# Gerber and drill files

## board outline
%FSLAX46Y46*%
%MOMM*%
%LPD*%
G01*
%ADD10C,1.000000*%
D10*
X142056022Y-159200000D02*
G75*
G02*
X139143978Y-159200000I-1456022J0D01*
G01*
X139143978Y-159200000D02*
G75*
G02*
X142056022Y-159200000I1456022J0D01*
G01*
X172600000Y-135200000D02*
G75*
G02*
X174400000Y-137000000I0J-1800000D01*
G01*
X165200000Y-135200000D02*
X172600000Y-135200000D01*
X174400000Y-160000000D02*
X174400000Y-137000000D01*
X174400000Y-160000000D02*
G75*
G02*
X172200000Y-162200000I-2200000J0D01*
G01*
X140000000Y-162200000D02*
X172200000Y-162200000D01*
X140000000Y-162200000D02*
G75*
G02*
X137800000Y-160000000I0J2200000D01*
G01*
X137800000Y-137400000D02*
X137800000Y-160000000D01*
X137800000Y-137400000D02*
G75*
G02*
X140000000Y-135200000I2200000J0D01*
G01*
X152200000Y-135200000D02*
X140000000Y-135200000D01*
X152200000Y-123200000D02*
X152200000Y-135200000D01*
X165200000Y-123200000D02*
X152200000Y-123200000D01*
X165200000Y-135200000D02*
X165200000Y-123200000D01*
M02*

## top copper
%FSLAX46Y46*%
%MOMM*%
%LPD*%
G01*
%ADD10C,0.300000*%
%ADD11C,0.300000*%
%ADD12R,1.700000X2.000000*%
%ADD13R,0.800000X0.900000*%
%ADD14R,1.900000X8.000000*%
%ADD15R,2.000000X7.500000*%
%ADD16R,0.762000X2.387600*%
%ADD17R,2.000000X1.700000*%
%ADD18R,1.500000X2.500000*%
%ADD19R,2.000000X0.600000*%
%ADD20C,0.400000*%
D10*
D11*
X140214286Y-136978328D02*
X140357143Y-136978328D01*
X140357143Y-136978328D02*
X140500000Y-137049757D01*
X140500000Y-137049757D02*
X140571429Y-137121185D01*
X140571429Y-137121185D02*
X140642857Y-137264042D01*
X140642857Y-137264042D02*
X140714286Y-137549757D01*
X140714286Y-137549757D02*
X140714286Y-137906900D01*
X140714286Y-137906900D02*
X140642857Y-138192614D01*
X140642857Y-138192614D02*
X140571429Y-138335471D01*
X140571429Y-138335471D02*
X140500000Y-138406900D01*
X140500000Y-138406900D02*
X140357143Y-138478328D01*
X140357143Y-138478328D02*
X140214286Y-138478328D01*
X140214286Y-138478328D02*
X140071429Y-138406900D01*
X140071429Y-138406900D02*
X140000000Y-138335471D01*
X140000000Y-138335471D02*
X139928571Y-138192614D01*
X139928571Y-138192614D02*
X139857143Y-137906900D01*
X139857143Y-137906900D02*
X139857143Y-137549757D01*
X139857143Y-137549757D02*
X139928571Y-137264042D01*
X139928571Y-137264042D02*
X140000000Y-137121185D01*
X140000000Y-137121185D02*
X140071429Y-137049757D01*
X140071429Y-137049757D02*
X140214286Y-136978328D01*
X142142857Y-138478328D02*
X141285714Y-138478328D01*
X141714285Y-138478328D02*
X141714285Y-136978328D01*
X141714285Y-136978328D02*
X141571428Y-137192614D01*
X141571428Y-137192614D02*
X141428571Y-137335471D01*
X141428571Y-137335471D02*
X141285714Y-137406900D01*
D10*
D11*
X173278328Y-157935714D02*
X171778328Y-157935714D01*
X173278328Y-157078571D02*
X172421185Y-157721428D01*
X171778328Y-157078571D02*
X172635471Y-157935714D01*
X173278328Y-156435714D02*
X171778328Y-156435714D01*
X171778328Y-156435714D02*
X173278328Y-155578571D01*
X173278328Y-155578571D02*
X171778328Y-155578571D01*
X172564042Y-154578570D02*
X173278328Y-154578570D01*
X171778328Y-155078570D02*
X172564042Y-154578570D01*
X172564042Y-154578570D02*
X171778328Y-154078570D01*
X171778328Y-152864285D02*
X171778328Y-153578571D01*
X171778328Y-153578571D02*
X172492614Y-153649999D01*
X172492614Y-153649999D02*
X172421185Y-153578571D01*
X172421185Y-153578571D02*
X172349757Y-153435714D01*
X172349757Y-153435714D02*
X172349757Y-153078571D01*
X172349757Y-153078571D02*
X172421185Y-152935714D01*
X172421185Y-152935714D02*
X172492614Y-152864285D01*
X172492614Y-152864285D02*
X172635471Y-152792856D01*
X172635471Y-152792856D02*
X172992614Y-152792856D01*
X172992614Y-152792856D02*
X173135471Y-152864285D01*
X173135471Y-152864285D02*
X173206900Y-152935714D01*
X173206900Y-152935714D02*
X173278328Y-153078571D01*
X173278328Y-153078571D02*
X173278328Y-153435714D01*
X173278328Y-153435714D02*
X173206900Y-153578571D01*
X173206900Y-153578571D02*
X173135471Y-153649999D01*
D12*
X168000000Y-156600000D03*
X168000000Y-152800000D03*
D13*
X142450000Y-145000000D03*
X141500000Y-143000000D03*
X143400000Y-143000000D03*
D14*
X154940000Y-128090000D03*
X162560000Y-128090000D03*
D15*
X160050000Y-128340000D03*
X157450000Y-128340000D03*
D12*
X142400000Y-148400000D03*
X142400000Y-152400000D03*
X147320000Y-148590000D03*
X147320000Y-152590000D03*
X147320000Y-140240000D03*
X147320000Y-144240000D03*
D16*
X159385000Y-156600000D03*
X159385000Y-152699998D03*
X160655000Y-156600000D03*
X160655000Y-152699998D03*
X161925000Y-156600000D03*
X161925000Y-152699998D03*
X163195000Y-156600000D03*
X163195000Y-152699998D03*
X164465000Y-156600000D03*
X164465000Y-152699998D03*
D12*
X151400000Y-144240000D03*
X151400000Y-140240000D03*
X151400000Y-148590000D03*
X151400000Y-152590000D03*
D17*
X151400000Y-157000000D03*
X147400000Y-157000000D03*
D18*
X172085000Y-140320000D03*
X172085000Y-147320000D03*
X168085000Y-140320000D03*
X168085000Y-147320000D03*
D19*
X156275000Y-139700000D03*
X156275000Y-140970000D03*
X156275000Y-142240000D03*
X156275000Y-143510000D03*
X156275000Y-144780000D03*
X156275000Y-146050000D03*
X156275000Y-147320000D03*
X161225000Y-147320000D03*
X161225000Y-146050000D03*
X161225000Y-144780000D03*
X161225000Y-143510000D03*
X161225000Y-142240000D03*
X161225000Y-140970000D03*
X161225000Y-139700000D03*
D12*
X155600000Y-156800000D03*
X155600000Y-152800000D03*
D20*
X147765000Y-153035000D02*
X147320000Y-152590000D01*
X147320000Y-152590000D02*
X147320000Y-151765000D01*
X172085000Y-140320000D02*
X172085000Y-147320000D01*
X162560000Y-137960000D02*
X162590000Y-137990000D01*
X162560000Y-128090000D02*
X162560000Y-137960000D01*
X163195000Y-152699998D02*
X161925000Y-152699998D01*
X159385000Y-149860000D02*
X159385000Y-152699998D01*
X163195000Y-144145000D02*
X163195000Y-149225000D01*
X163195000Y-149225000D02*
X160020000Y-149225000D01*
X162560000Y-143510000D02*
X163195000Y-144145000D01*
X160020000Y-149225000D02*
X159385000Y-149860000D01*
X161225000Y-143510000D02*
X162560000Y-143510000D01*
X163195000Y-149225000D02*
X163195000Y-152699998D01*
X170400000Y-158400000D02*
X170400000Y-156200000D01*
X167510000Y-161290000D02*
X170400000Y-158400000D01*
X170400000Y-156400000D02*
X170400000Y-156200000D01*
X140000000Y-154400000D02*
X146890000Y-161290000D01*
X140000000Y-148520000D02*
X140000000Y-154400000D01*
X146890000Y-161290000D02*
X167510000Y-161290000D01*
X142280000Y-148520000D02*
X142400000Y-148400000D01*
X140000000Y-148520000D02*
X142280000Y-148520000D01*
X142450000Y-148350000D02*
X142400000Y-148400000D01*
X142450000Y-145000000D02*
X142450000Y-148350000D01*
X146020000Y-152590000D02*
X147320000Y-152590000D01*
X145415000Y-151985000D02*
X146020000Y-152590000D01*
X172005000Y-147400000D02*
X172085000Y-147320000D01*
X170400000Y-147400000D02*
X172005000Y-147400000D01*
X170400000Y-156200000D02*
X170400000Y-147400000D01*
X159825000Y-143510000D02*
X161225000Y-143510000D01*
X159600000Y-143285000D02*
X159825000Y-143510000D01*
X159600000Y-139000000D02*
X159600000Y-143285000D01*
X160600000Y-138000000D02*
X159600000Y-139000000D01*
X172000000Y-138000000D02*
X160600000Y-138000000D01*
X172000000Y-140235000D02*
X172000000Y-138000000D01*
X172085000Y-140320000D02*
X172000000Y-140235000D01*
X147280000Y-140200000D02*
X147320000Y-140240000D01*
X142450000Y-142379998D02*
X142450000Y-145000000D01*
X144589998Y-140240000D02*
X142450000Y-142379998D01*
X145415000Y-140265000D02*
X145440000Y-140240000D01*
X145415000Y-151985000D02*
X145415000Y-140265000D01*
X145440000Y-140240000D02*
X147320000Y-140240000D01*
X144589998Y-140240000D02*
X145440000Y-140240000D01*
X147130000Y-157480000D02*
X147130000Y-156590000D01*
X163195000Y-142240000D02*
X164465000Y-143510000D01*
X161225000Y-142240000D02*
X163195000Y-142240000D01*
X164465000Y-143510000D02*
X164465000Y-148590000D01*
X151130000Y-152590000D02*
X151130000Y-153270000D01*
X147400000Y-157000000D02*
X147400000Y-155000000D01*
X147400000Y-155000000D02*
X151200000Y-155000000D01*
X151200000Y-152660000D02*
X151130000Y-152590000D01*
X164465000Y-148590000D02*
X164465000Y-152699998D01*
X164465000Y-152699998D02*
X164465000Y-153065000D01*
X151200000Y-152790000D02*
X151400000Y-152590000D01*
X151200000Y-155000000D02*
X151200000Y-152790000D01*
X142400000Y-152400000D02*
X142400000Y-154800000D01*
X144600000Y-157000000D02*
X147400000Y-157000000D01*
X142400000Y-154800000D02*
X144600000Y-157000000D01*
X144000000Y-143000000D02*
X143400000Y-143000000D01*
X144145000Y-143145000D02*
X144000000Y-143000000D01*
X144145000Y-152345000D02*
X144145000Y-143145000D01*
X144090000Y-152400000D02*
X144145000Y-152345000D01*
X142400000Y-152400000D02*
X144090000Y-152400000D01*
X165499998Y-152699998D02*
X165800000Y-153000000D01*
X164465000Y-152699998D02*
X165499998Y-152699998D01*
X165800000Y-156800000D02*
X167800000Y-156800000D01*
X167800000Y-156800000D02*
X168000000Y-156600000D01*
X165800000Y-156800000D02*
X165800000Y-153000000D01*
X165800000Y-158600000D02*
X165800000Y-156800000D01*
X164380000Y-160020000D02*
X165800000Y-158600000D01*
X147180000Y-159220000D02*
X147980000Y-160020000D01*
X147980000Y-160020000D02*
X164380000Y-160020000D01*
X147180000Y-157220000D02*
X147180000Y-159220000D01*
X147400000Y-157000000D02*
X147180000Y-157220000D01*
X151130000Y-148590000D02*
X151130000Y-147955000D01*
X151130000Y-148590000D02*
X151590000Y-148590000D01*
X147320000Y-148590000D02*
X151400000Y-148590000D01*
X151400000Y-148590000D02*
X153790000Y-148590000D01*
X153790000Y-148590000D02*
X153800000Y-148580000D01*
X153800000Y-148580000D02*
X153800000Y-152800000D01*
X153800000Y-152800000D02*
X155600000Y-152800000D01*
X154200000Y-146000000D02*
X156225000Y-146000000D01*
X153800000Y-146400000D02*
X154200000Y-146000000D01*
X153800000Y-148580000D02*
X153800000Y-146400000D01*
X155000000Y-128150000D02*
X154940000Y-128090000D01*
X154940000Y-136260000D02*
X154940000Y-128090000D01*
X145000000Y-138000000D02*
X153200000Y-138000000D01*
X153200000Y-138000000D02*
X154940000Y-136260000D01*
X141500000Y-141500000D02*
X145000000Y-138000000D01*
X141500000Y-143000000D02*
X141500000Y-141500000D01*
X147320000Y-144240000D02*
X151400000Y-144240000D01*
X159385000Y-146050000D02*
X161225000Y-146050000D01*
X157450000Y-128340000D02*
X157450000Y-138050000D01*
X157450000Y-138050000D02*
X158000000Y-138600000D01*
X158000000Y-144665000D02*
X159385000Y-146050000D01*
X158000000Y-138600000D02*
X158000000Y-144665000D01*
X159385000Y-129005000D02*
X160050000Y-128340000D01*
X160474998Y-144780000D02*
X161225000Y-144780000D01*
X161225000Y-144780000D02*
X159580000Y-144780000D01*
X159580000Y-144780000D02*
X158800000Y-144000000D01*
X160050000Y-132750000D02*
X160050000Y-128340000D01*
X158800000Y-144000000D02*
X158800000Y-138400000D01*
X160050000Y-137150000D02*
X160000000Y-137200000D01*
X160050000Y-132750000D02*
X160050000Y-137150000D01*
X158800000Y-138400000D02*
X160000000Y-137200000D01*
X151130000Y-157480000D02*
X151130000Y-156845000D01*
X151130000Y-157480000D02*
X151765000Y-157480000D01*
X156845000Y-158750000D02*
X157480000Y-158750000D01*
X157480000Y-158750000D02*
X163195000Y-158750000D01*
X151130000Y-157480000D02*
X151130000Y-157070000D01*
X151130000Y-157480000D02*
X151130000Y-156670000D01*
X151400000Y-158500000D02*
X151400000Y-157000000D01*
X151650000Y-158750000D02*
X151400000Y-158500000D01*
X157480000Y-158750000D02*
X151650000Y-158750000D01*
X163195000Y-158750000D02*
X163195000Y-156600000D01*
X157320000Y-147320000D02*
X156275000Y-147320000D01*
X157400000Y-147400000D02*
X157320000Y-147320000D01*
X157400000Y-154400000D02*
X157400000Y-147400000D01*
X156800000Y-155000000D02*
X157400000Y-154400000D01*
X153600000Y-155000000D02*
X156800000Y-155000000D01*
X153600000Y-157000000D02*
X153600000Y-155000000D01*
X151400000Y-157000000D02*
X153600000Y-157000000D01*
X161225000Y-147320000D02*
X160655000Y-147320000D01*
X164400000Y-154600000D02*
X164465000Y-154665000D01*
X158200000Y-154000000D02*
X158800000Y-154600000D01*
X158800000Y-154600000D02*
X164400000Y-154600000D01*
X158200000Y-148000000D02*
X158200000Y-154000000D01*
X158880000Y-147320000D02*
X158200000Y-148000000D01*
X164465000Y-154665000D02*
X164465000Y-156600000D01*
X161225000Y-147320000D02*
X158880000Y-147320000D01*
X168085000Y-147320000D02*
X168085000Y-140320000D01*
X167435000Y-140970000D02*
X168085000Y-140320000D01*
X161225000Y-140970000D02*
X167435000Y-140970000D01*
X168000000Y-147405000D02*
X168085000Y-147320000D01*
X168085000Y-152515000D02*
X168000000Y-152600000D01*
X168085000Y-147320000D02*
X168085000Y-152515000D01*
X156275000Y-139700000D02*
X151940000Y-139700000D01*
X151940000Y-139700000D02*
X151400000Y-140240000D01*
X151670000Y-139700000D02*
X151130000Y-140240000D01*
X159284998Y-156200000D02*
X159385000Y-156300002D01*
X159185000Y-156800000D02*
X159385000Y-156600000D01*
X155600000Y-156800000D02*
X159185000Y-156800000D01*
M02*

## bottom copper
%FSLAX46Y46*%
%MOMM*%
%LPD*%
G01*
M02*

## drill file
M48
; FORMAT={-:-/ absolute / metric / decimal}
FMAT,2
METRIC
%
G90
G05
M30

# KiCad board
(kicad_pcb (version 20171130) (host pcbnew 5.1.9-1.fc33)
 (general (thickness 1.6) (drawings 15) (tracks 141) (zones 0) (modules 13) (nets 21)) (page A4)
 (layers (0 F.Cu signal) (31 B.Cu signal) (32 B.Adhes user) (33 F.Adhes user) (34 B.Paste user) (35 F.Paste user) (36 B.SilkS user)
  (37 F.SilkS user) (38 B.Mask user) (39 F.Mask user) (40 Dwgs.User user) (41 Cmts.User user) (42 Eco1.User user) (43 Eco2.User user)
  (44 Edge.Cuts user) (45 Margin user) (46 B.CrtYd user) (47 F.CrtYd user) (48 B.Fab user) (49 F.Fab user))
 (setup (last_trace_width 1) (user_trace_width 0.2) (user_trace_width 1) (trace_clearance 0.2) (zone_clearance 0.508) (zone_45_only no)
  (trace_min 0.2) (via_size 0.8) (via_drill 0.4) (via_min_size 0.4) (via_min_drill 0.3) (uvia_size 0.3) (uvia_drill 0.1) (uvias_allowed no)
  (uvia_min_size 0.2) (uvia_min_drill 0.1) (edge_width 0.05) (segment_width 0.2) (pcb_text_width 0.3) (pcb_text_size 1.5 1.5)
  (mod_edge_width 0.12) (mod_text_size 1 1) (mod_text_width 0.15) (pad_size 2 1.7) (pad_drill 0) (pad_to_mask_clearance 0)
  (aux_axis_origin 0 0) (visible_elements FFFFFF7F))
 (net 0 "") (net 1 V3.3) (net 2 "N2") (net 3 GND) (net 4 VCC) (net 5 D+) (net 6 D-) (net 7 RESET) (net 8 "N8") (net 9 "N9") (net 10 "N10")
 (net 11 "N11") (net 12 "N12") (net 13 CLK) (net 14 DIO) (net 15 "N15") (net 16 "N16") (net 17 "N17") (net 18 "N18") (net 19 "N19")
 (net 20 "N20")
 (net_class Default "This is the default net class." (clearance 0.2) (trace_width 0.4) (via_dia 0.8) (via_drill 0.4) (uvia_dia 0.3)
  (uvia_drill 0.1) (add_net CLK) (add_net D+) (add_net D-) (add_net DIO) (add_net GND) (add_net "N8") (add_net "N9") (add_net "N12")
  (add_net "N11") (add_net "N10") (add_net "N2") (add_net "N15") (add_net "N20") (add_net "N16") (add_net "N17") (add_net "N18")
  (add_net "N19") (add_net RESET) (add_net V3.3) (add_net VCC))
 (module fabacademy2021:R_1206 (layer F.Cu) (at 168 154.6 90)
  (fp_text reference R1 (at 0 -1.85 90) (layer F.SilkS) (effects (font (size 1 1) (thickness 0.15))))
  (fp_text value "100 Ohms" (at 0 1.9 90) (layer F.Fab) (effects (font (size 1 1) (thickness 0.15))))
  (pad 1 smd rect (at -2 0 90) (size 2 1.7) (layers F.Cu F.Paste F.Mask) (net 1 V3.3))
  (pad 2 smd rect (at 1.8 0 90) (size 2 1.7) (layers F.Cu F.Paste F.Mask) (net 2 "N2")))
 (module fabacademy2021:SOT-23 (layer F.Cu) (at 142.45 144 270)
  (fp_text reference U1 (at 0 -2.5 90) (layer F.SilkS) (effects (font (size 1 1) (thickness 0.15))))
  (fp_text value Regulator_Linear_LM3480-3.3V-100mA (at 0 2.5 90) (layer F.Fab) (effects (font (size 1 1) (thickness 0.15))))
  (pad 3 smd rect (at 1 0 270) (size 0.9 0.8) (layers F.Cu F.Paste F.Mask) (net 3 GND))
  (pad 2 smd rect (at -1 0.95 270) (size 0.9 0.8) (layers F.Cu F.Paste F.Mask) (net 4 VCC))
  (pad 1 smd rect (at -1 -0.95 270) (size 0.9 0.8) (layers F.Cu F.Paste F.Mask) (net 1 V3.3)))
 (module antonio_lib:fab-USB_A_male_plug (layer F.Cu) (at 158.75 123.19 180)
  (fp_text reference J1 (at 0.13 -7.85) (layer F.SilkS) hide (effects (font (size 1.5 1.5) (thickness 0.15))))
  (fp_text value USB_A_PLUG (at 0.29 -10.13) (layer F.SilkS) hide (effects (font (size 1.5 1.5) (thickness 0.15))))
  (pad 1 connect rect (at 3.81 -4.9 180) (size 1.9 8) (layers F.Cu F.Mask) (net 4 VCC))
  (pad 4 connect rect (at -3.81 -4.9 180) (size 1.9 8) (layers F.Cu F.Mask) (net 3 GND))
  (pad 3 connect rect (at -1.3 -5.15 180) (size 2 7.5) (layers F.Cu F.Mask) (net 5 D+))
  (pad 2 connect rect (at 1.3 -5.15 180) (size 2 7.5) (layers F.Cu F.Mask) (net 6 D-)))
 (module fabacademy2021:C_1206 (layer F.Cu) (at 142.4 150.4 90)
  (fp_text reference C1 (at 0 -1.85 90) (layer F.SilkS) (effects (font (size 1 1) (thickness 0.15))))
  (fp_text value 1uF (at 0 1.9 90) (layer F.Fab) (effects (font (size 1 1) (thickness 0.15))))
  (pad 2 smd rect (at 2 0 90) (size 2 1.7) (layers F.Cu F.Paste F.Mask) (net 3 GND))
  (pad 1 smd rect (at -2 0 90) (size 2 1.7) (layers F.Cu F.Paste F.Mask) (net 1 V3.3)))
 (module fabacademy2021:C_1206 (layer F.Cu) (at 147.32 150.59 270)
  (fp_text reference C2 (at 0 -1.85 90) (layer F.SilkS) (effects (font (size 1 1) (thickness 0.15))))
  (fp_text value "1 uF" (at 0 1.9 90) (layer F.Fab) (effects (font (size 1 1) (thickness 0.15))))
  (pad 1 smd rect (at -2 0 270) (size 2 1.7) (layers F.Cu F.Paste F.Mask) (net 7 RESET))
  (pad 2 smd rect (at 2 0 270) (size 2 1.7) (layers F.Cu F.Paste F.Mask) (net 3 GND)))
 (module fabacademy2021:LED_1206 (layer F.Cu) (at 147.32 142.24 90)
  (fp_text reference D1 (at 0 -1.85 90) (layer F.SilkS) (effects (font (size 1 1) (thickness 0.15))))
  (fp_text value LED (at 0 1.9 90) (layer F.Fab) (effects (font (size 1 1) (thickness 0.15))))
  (pad 2 smd rect (at 2 0 90) (size 2 1.7) (layers F.Cu F.Paste F.Mask) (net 3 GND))
  (pad 1 smd rect (at -2 0 90) (size 2 1.7) (layers F.Cu F.Paste F.Mask) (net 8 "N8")))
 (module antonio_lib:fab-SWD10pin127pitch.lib (layer F.Cu) (at 159.385 156.599999 180)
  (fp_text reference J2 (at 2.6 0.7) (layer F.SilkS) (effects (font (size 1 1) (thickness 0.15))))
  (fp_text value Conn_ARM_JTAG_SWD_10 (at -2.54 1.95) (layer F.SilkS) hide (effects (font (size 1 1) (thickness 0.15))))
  (pad 10 smd rect (at 0 -0.000001 180) (size 0.762 2.3876) (layers F.Cu F.Paste F.Mask) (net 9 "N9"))
  (pad 9 smd rect (at 0 3.900001 180) (size 0.762 2.3876) (layers F.Cu F.Paste F.Mask) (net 3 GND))
  (pad 8 smd rect (at -1.27 -0.000001 180) (size 0.762 2.3876) (layers F.Cu F.Paste F.Mask) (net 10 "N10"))
  (pad 7 smd rect (at -1.27 3.900001 180) (size 0.762 2.3876) (layers F.Cu F.Paste F.Mask) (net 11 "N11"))
  (pad 6 smd rect (at -2.54 -0.000001 180) (size 0.762 2.3876) (layers F.Cu F.Paste F.Mask) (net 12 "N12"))
  (pad 5 smd rect (at -2.54 3.900001 180) (size 0.762 2.3876) (layers F.Cu F.Paste F.Mask) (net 3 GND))
  (pad 4 smd rect (at -3.81 -0.000001 180) (size 0.762 2.3876) (layers F.Cu F.Paste F.Mask) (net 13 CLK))
  (pad 3 smd rect (at -3.81 3.900001 180) (size 0.762 2.3876) (layers F.Cu F.Paste F.Mask) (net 3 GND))
  (pad 2 smd rect (at -5.08 -0.000001 180) (size 0.762 2.3876) (layers F.Cu F.Paste F.Mask) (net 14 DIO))
  (pad 1 smd rect (at -5.08 3.900001 180) (size 0.762 2.3876) (layers F.Cu F.Paste F.Mask) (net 1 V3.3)))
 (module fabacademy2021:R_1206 (layer F.Cu) (at 151.4 142.24 270)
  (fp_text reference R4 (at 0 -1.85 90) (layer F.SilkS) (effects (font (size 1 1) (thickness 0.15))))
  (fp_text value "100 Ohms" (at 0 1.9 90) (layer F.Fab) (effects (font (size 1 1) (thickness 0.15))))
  (pad 2 smd rect (at 2 0 270) (size 2 1.7) (layers F.Cu F.Paste F.Mask) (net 8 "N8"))
  (pad 1 smd rect (at -2 0 270) (size 2 1.7) (layers F.Cu F.Paste F.Mask) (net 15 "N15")))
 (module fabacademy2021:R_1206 (layer F.Cu) (at 151.4 150.59 270)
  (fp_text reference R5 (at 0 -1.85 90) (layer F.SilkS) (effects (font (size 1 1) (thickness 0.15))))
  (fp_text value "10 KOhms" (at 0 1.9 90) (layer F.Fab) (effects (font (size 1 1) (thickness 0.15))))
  (pad 1 smd rect (at -2 0 270) (size 2 1.7) (layers F.Cu F.Paste F.Mask) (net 7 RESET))
  (pad 2 smd rect (at 2 0 270) (size 2 1.7) (layers F.Cu F.Paste F.Mask) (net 1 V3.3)))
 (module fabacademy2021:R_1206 (layer F.Cu) (at 149.4 157 180)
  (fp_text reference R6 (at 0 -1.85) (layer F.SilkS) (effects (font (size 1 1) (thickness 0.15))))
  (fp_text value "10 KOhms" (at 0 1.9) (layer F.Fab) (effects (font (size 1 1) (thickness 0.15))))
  (pad 1 smd rect (at -2 0 180) (size 2 1.7) (layers F.Cu F.Paste F.Mask) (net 13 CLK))
  (pad 2 smd rect (at 2 0 180) (size 2 1.7) (layers F.Cu F.Paste F.Mask) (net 1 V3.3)))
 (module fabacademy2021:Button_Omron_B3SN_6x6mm (layer F.Cu) (at 170.085 143.82 90)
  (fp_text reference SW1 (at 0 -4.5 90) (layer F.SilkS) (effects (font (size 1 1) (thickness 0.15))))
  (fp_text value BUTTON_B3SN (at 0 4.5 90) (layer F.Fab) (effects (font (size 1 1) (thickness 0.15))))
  (pad 2 smd rect (at 3.5 2 90) (size 2.5 1.5) (layers F.Cu F.Paste F.Mask) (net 3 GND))
  (pad 2 smd rect (at -3.5 2 90) (size 2.5 1.5) (layers F.Cu F.Paste F.Mask) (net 3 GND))
  (pad 1 smd rect (at 3.5 -2 90) (size 2.5 1.5) (layers F.Cu F.Paste F.Mask) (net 2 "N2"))
  (pad 1 smd rect (at -3.5 -2 90) (size 2.5 1.5) (layers F.Cu F.Paste F.Mask) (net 2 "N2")))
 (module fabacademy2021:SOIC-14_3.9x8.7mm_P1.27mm (layer F.Cu) (at 158.75 143.51)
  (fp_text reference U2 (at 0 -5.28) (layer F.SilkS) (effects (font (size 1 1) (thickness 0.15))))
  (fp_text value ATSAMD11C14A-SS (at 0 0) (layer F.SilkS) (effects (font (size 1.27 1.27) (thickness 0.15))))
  (pad 1 smd rect (at -2.475 -3.81) (size 2 0.6) (layers F.Cu F.Paste F.Mask) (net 15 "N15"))
  (pad 2 smd rect (at -2.475 -2.54) (size 2 0.6) (layers F.Cu F.Paste F.Mask) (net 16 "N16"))
  (pad 3 smd rect (at -2.475 -1.27) (size 2 0.6) (layers F.Cu F.Paste F.Mask) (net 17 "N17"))
  (pad 4 smd rect (at -2.475 0) (size 2 0.6) (layers F.Cu F.Paste F.Mask) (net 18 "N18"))
  (pad 5 smd rect (at -2.475 1.27) (size 2 0.6) (layers F.Cu F.Paste F.Mask) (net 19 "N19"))
  (pad 6 smd rect (at -2.475 2.54) (size 2 0.6) (layers F.Cu F.Paste F.Mask) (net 7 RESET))
  (pad 7 smd rect (at -2.475 3.81) (size 2 0.6) (layers F.Cu F.Paste F.Mask) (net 13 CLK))
  (pad 8 smd rect (at 2.475 3.81) (size 2 0.6) (layers F.Cu F.Paste F.Mask) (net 14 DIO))
  (pad 9 smd rect (at 2.475 2.54) (size 2 0.6) (layers F.Cu F.Paste F.Mask) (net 6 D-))
  (pad 10 smd rect (at 2.475 1.27) (size 2 0.6) (layers F.Cu F.Paste F.Mask) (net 5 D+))
  (pad 11 smd rect (at 2.475 0) (size 2 0.6) (layers F.Cu F.Paste F.Mask) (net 3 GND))
  (pad 12 smd rect (at 2.475 -1.27) (size 2 0.6) (layers F.Cu F.Paste F.Mask) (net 1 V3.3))
  (pad 13 smd rect (at 2.475 -2.54) (size 2 0.6) (layers F.Cu F.Paste F.Mask) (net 2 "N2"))
  (pad 14 smd rect (at 2.475 -3.81) (size 2 0.6) (layers F.Cu F.Paste F.Mask) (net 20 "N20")))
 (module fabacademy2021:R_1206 (layer F.Cu) (at 155.6 154.8 270)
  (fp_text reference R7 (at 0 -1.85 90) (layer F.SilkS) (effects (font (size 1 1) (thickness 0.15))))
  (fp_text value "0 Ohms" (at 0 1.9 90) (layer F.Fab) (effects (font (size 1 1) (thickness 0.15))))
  (pad 2 smd rect (at 2 0 270) (size 2 1.7) (layers F.Cu F.Paste F.Mask) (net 9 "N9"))
  (pad 1 smd rect (at -2 0 270) (size 2 1.7) (layers F.Cu F.Paste F.Mask) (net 7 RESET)))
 (gr_circle (center 140.6 159.2) (end 142.056022 159.2) (layer Edge.Cuts) (width 1))
 (gr_arc (start 172.6 137) (end 174.4 137) (angle -90) (layer Edge.Cuts) (width 1))
 (gr_line (start 165.2 135.2) (end 172.6 135.2) (layer Edge.Cuts) (width 1))
 (gr_line (start 174.4 160) (end 174.4 137) (layer Edge.Cuts) (width 1))
 (gr_arc (start 172.2 160) (end 172.2 162.2) (angle -90) (layer Edge.Cuts) (width 1))
 (gr_line (start 140 162.2) (end 172.2 162.2) (layer Edge.Cuts) (width 1))
 (gr_arc (start 140 160) (end 137.8 160) (angle -90) (layer Edge.Cuts) (width 1))
 (gr_line (start 137.8 137.4) (end 137.8 160) (layer Edge.Cuts) (width 1))
 (gr_arc (start 140 137.4) (end 140 135.2) (angle -90) (layer Edge.Cuts) (width 1))
 (gr_line (start 152.2 135.2) (end 140 135.2) (layer Edge.Cuts) (width 1))
 (gr_line (start 152.2 123.2) (end 152.2 135.2) (layer Edge.Cuts) (width 1))
 (gr_line (start 165.2 123.2) (end 152.2 123.2) (layer Edge.Cuts) (width 1))
 (gr_line (start 165.2 135.2) (end 165.2 123.2) (layer Edge.Cuts) (width 1))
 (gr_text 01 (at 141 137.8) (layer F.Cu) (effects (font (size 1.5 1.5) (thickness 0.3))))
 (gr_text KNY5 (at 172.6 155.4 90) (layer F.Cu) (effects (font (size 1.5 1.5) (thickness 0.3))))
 (segment (start 147.765 153.035) (end 147.32 152.59) (width 0.4) (layer F.Cu) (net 3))
 (segment (start 147.32 152.59) (end 147.32 151.765) (width 0.4) (layer F.Cu) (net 3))
 (segment (start 172.085 140.32) (end 172.085 147.32) (width 0.4) (layer F.Cu) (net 3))
 (segment (start 162.56 137.96) (end 162.59 137.99) (width 0.4) (layer F.Cu) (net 3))
 (segment (start 162.56 128.09) (end 162.56 137.96) (width 0.4) (layer F.Cu) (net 3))
 (segment (start 163.195 152.699998) (end 161.925 152.699998) (width 0.4) (layer F.Cu) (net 3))
 (segment (start 159.385 149.86) (end 159.385 152.699998) (width 0.4) (layer F.Cu) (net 3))
 (segment (start 163.195 144.145) (end 163.195 149.225) (width 0.4) (layer F.Cu) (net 3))
 (segment (start 163.195 149.225) (end 160.02 149.225) (width 0.4) (layer F.Cu) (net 3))
 (segment (start 162.56 143.51) (end 163.195 144.145) (width 0.4) (layer F.Cu) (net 3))
 (segment (start 160.02 149.225) (end 159.385 149.86) (width 0.4) (layer F.Cu) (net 3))
 (segment (start 161.225 143.51) (end 162.56 143.51) (width 0.4) (layer F.Cu) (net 3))
 (segment (start 163.195 149.225) (end 163.195 152.699998) (width 0.4) (layer F.Cu) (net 3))
 (segment (start 170.4 158.4) (end 170.4 156.2) (width 0.4) (layer F.Cu) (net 3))
 (segment (start 167.51 161.29) (end 170.4 158.4) (width 0.4) (layer F.Cu) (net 3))
 (segment (start 170.4 156.4) (end 170.4 156.2) (width 0.4) (layer F.Cu) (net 3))
 (segment (start 140 154.4) (end 146.89 161.29) (width 0.4) (layer F.Cu) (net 3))
 (segment (start 140 148.52) (end 140 154.4) (width 0.4) (layer F.Cu) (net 3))
 (segment (start 146.89 161.29) (end 167.51 161.29) (width 0.4) (layer F.Cu) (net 3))
 (segment (start 142.28 148.52) (end 142.4 148.4) (width 0.4) (layer F.Cu) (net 3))
 (segment (start 140 148.52) (end 142.28 148.52) (width 0.4) (layer F.Cu) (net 3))
 (segment (start 142.45 148.35) (end 142.4 148.4) (width 0.4) (layer F.Cu) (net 3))
 (segment (start 142.45 145) (end 142.45 148.35) (width 0.4) (layer F.Cu) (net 3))
 (segment (start 146.02 152.59) (end 147.32 152.59) (width 0.4) (layer F.Cu) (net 3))
 (segment (start 145.415 151.985) (end 146.02 152.59) (width 0.4) (layer F.Cu) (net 3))
 (segment (start 172.005 147.4) (end 172.085 147.32) (width 0.4) (layer F.Cu) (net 3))
 (segment (start 170.4 147.4) (end 172.005 147.4) (width 0.4) (layer F.Cu) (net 3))
 (segment (start 170.4 156.2) (end 170.4 147.4) (width 0.4) (layer F.Cu) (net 3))
 (segment (start 159.825 143.51) (end 161.225 143.51) (width 0.4) (layer F.Cu) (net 3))
 (segment (start 159.6 143.285) (end 159.825 143.51) (width 0.4) (layer F.Cu) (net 3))
 (segment (start 159.6 139) (end 159.6 143.285) (width 0.4) (layer F.Cu) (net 3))
 (segment (start 160.6 138) (end 159.6 139) (width 0.4) (layer F.Cu) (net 3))
 (segment (start 172 138) (end 160.6 138) (width 0.4) (layer F.Cu) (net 3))
 (segment (start 172 140.235) (end 172 138) (width 0.4) (layer F.Cu) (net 3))
 (segment (start 172.085 140.32) (end 172 140.235) (width 0.4) (layer F.Cu) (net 3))
 (segment (start 147.28 140.2) (end 147.32 140.24) (width 0.4) (layer F.Cu) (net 3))
 (segment (start 142.45 142.379998) (end 142.45 145) (width 0.4) (layer F.Cu) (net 3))
 (segment (start 144.589998 140.24) (end 142.45 142.379998) (width 0.4) (layer F.Cu) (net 3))
 (segment (start 145.415 140.265) (end 145.44 140.24) (width 0.4) (layer F.Cu) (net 3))
 (segment (start 145.415 151.985) (end 145.415 140.265) (width 0.4) (layer F.Cu) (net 3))
 (segment (start 145.44 140.24) (end 147.32 140.24) (width 0.4) (layer F.Cu) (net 3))
 (segment (start 144.589998 140.24) (end 145.44 140.24) (width 0.4) (layer F.Cu) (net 3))
 (segment (start 147.13 157.48) (end 147.13 156.59) (width 0.4) (layer F.Cu) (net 1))
 (segment (start 163.195 142.24) (end 164.465 143.51) (width 0.4) (layer F.Cu) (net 1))
 (segment (start 161.225 142.24) (end 163.195 142.24) (width 0.4) (layer F.Cu) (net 1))
 (segment (start 164.465 143.51) (end 164.465 148.59) (width 0.4) (layer F.Cu) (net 1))
 (segment (start 151.13 152.59) (end 151.13 153.27) (width 0.4) (layer F.Cu) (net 1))
 (segment (start 147.4 157) (end 147.4 155) (width 0.4) (layer F.Cu) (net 1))
 (segment (start 147.4 155) (end 151.2 155) (width 0.4) (layer F.Cu) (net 1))
 (segment (start 151.2 152.66) (end 151.13 152.59) (width 0.4) (layer F.Cu) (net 1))
 (segment (start 164.465 148.59) (end 164.465 152.699998) (width 0.4) (layer F.Cu) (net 1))
 (segment (start 164.465 152.699998) (end 164.465 153.065) (width 0.4) (layer F.Cu) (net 1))
 (segment (start 151.2 152.79) (end 151.4 152.59) (width 0.4) (layer F.Cu) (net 1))
 (segment (start 151.2 155) (end 151.2 152.79) (width 0.4) (layer F.Cu) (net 1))
 (segment (start 142.4 152.4) (end 142.4 154.8) (width 0.4) (layer F.Cu) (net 1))
 (segment (start 144.6 157) (end 147.4 157) (width 0.4) (layer F.Cu) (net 1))
 (segment (start 142.4 154.8) (end 144.6 157) (width 0.4) (layer F.Cu) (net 1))
 (segment (start 144 143) (end 143.4 143) (width 0.4) (layer F.Cu) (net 1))
 (segment (start 144.145 143.145) (end 144 143) (width 0.4) (layer F.Cu) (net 1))
 (segment (start 144.145 152.345) (end 144.145 143.145) (width 0.4) (layer F.Cu) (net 1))
 (segment (start 144.09 152.4) (end 144.145 152.345) (width 0.4) (layer F.Cu) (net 1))
 (segment (start 142.4 152.4) (end 144.09 152.4) (width 0.4) (layer F.Cu) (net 1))
 (segment (start 165.499998 152.699998) (end 165.8 153) (width 0.4) (layer F.Cu) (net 1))
 (segment (start 164.465 152.699998) (end 165.499998 152.699998) (width 0.4) (layer F.Cu) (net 1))
 (segment (start 165.8 156.8) (end 167.8 156.8) (width 0.4) (layer F.Cu) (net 1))
 (segment (start 167.8 156.8) (end 168 156.6) (width 0.4) (layer F.Cu) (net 1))
 (segment (start 165.8 156.8) (end 165.8 153) (width 0.4) (layer F.Cu) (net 1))
 (segment (start 165.8 158.6) (end 165.8 156.8) (width 0.4) (layer F.Cu) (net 1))
 (segment (start 164.38 160.02) (end 165.8 158.6) (width 0.4) (layer F.Cu) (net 1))
 (segment (start 147.18 159.22) (end 147.98 160.02) (width 0.4) (layer F.Cu) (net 1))
 (segment (start 147.98 160.02) (end 164.38 160.02) (width 0.4) (layer F.Cu) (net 1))
 (segment (start 147.18 157.22) (end 147.18 159.22) (width 0.4) (layer F.Cu) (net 1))
 (segment (start 147.4 157) (end 147.18 157.22) (width 0.4) (layer F.Cu) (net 1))
 (segment (start 151.13 148.59) (end 151.13 147.955) (width 0.4) (layer F.Cu) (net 7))
 (segment (start 151.13 148.59) (end 151.59 148.59) (width 0.4) (layer F.Cu) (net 7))
 (segment (start 147.32 148.59) (end 151.4 148.59) (width 0.4) (layer F.Cu) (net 7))
 (segment (start 151.4 148.59) (end 153.79 148.59) (width 0.4) (layer F.Cu) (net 7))
 (segment (start 153.79 148.59) (end 153.8 148.58) (width 0.4) (layer F.Cu) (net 7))
 (segment (start 153.8 148.58) (end 153.8 152.8) (width 0.4) (layer F.Cu) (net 7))
 (segment (start 153.8 152.8) (end 155.6 152.8) (width 0.4) (layer F.Cu) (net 7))
 (segment (start 154.2 146) (end 156.225 146) (width 0.4) (layer F.Cu) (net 7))
 (segment (start 153.8 146.4) (end 154.2 146) (width 0.4) (layer F.Cu) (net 7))
 (segment (start 153.8 148.58) (end 153.8 146.4) (width 0.4) (layer F.Cu) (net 7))
 (segment (start 155 128.15) (end 154.94 128.09) (width 0.4) (layer F.Cu) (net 4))
 (segment (start 154.94 136.26) (end 154.94 128.09) (width 0.4) (layer F.Cu) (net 4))
 (segment (start 145 138) (end 153.2 138) (width 0.4) (layer F.Cu) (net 4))
 (segment (start 153.2 138) (end 154.94 136.26) (width 0.4) (layer F.Cu) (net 4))
 (segment (start 141.5 141.5) (end 145 138) (width 0.4) (layer F.Cu) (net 4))
 (segment (start 141.5 143) (end 141.5 141.5) (width 0.4) (layer F.Cu) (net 4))
 (segment (start 147.32 144.24) (end 151.4 144.24) (width 0.4) (layer F.Cu) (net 8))
 (segment (start 159.385 146.05) (end 161.225 146.05) (width 0.4) (layer F.Cu) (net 6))
 (segment (start 157.45 128.34) (end 157.45 138.05) (width 0.4) (layer F.Cu) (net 6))
 (segment (start 157.45 138.05) (end 158 138.6) (width 0.4) (layer F.Cu) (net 6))
 (segment (start 158 144.665) (end 159.385 146.05) (width 0.4) (layer F.Cu) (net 6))
 (segment (start 158 138.6) (end 158 144.665) (width 0.4) (layer F.Cu) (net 6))
 (segment (start 159.385 129.005) (end 160.05 128.34) (width 0.4) (layer F.Cu) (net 5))
 (segment (start 160.474998 144.78) (end 161.225 144.78) (width 0.4) (layer F.Cu) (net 5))
 (segment (start 161.225 144.78) (end 159.58 144.78) (width 0.4) (layer F.Cu) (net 5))
 (segment (start 159.58 144.78) (end 158.8 144) (width 0.4) (layer F.Cu) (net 5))
 (segment (start 160.05 132.75) (end 160.05 128.34) (width 0.4) (layer F.Cu) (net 5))
 (segment (start 158.8 144) (end 158.8 138.4) (width 0.4) (layer F.Cu) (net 5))
 (segment (start 160.05 137.15) (end 160 137.2) (width 0.4) (layer F.Cu) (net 5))
 (segment (start 160.05 132.75) (end 160.05 137.15) (width 0.4) (layer F.Cu) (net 5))
 (segment (start 158.8 138.4) (end 160 137.2) (width 0.4) (layer F.Cu) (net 5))
 (segment (start 151.13 157.48) (end 151.13 156.845) (width 0.4) (layer F.Cu) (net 13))
 (segment (start 151.13 157.48) (end 151.765 157.48) (width 0.4) (layer F.Cu) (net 13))
 (segment (start 156.845 158.75) (end 157.48 158.75) (width 0.4) (layer F.Cu) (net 13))
 (segment (start 157.48 158.75) (end 163.195 158.75) (width 0.4) (layer F.Cu) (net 13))
 (segment (start 151.13 157.48) (end 151.13 157.07) (width 0.4) (layer F.Cu) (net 13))
 (segment (start 151.13 157.48) (end 151.13 156.67) (width 0.4) (layer F.Cu) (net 13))
 (segment (start 151.4 158.5) (end 151.4 157) (width 0.4) (layer F.Cu) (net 13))
 (segment (start 151.65 158.75) (end 151.4 158.5) (width 0.4) (layer F.Cu) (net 13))
 (segment (start 157.48 158.75) (end 151.65 158.75) (width 0.4) (layer F.Cu) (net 13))
 (segment (start 163.195 158.75) (end 163.195 156.6) (width 0.4) (layer F.Cu) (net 13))
 (segment (start 157.32 147.32) (end 156.275 147.32) (width 0.4) (layer F.Cu) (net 13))
 (segment (start 157.4 147.4) (end 157.32 147.32) (width 0.4) (layer F.Cu) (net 13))
 (segment (start 157.4 154.4) (end 157.4 147.4) (width 0.4) (layer F.Cu) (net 13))
 (segment (start 156.8 155) (end 157.4 154.4) (width 0.4) (layer F.Cu) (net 13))
 (segment (start 153.6 155) (end 156.8 155) (width 0.4) (layer F.Cu) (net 13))
 (segment (start 153.6 157) (end 153.6 155) (width 0.4) (layer F.Cu) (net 13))
 (segment (start 151.4 157) (end 153.6 157) (width 0.4) (layer F.Cu) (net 13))
 (segment (start 161.225 147.32) (end 160.655 147.32) (width 0.4) (layer F.Cu) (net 14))
 (segment (start 164.4 154.6) (end 164.465 154.665) (width 0.4) (layer F.Cu) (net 14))
 (segment (start 158.2 154) (end 158.8 154.6) (width 0.4) (layer F.Cu) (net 14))
 (segment (start 158.8 154.6) (end 164.4 154.6) (width 0.4) (layer F.Cu) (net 14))
 (segment (start 158.2 148) (end 158.2 154) (width 0.4) (layer F.Cu) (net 14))
 (segment (start 158.88 147.32) (end 158.2 148) (width 0.4) (layer F.Cu) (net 14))
 (segment (start 164.465 154.665) (end 164.465 156.6) (width 0.4) (layer F.Cu) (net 14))
 (segment (start 161.225 147.32) (end 158.88 147.32) (width 0.4) (layer F.Cu) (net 14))
 (segment (start 168.085 147.32) (end 168.085 140.32) (width 0.4) (layer F.Cu) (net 2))
 (segment (start 167.435 140.97) (end 168.085 140.32) (width 0.4) (layer F.Cu) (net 2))
 (segment (start 161.225 140.97) (end 167.435 140.97) (width 0.4) (layer F.Cu) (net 2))
 (segment (start 168 147.405) (end 168.085 147.32) (width 0.4) (layer F.Cu) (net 2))
 (segment (start 168.085 152.515) (end 168 152.6) (width 0.4) (layer F.Cu) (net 2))
 (segment (start 168.085 147.32) (end 168.085 152.515) (width 0.4) (layer F.Cu) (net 2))
 (segment (start 156.275 139.7) (end 151.94 139.7) (width 0.4) (layer F.Cu) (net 15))
 (segment (start 151.94 139.7) (end 151.4 140.24) (width 0.4) (layer F.Cu) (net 15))
 (segment (start 151.67 139.7) (end 151.13 140.24) (width 0.4) (layer F.Cu) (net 15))
 (segment (start 159.284998 156.2) (end 159.385 156.300002) (width 0.4) (layer F.Cu) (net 9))
 (segment (start 159.185 156.8) (end 159.385 156.6) (width 0.4) (layer F.Cu) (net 9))
 (segment (start 155.6 156.8) (end 159.185 156.8) (width 0.4) (layer F.Cu) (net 9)))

